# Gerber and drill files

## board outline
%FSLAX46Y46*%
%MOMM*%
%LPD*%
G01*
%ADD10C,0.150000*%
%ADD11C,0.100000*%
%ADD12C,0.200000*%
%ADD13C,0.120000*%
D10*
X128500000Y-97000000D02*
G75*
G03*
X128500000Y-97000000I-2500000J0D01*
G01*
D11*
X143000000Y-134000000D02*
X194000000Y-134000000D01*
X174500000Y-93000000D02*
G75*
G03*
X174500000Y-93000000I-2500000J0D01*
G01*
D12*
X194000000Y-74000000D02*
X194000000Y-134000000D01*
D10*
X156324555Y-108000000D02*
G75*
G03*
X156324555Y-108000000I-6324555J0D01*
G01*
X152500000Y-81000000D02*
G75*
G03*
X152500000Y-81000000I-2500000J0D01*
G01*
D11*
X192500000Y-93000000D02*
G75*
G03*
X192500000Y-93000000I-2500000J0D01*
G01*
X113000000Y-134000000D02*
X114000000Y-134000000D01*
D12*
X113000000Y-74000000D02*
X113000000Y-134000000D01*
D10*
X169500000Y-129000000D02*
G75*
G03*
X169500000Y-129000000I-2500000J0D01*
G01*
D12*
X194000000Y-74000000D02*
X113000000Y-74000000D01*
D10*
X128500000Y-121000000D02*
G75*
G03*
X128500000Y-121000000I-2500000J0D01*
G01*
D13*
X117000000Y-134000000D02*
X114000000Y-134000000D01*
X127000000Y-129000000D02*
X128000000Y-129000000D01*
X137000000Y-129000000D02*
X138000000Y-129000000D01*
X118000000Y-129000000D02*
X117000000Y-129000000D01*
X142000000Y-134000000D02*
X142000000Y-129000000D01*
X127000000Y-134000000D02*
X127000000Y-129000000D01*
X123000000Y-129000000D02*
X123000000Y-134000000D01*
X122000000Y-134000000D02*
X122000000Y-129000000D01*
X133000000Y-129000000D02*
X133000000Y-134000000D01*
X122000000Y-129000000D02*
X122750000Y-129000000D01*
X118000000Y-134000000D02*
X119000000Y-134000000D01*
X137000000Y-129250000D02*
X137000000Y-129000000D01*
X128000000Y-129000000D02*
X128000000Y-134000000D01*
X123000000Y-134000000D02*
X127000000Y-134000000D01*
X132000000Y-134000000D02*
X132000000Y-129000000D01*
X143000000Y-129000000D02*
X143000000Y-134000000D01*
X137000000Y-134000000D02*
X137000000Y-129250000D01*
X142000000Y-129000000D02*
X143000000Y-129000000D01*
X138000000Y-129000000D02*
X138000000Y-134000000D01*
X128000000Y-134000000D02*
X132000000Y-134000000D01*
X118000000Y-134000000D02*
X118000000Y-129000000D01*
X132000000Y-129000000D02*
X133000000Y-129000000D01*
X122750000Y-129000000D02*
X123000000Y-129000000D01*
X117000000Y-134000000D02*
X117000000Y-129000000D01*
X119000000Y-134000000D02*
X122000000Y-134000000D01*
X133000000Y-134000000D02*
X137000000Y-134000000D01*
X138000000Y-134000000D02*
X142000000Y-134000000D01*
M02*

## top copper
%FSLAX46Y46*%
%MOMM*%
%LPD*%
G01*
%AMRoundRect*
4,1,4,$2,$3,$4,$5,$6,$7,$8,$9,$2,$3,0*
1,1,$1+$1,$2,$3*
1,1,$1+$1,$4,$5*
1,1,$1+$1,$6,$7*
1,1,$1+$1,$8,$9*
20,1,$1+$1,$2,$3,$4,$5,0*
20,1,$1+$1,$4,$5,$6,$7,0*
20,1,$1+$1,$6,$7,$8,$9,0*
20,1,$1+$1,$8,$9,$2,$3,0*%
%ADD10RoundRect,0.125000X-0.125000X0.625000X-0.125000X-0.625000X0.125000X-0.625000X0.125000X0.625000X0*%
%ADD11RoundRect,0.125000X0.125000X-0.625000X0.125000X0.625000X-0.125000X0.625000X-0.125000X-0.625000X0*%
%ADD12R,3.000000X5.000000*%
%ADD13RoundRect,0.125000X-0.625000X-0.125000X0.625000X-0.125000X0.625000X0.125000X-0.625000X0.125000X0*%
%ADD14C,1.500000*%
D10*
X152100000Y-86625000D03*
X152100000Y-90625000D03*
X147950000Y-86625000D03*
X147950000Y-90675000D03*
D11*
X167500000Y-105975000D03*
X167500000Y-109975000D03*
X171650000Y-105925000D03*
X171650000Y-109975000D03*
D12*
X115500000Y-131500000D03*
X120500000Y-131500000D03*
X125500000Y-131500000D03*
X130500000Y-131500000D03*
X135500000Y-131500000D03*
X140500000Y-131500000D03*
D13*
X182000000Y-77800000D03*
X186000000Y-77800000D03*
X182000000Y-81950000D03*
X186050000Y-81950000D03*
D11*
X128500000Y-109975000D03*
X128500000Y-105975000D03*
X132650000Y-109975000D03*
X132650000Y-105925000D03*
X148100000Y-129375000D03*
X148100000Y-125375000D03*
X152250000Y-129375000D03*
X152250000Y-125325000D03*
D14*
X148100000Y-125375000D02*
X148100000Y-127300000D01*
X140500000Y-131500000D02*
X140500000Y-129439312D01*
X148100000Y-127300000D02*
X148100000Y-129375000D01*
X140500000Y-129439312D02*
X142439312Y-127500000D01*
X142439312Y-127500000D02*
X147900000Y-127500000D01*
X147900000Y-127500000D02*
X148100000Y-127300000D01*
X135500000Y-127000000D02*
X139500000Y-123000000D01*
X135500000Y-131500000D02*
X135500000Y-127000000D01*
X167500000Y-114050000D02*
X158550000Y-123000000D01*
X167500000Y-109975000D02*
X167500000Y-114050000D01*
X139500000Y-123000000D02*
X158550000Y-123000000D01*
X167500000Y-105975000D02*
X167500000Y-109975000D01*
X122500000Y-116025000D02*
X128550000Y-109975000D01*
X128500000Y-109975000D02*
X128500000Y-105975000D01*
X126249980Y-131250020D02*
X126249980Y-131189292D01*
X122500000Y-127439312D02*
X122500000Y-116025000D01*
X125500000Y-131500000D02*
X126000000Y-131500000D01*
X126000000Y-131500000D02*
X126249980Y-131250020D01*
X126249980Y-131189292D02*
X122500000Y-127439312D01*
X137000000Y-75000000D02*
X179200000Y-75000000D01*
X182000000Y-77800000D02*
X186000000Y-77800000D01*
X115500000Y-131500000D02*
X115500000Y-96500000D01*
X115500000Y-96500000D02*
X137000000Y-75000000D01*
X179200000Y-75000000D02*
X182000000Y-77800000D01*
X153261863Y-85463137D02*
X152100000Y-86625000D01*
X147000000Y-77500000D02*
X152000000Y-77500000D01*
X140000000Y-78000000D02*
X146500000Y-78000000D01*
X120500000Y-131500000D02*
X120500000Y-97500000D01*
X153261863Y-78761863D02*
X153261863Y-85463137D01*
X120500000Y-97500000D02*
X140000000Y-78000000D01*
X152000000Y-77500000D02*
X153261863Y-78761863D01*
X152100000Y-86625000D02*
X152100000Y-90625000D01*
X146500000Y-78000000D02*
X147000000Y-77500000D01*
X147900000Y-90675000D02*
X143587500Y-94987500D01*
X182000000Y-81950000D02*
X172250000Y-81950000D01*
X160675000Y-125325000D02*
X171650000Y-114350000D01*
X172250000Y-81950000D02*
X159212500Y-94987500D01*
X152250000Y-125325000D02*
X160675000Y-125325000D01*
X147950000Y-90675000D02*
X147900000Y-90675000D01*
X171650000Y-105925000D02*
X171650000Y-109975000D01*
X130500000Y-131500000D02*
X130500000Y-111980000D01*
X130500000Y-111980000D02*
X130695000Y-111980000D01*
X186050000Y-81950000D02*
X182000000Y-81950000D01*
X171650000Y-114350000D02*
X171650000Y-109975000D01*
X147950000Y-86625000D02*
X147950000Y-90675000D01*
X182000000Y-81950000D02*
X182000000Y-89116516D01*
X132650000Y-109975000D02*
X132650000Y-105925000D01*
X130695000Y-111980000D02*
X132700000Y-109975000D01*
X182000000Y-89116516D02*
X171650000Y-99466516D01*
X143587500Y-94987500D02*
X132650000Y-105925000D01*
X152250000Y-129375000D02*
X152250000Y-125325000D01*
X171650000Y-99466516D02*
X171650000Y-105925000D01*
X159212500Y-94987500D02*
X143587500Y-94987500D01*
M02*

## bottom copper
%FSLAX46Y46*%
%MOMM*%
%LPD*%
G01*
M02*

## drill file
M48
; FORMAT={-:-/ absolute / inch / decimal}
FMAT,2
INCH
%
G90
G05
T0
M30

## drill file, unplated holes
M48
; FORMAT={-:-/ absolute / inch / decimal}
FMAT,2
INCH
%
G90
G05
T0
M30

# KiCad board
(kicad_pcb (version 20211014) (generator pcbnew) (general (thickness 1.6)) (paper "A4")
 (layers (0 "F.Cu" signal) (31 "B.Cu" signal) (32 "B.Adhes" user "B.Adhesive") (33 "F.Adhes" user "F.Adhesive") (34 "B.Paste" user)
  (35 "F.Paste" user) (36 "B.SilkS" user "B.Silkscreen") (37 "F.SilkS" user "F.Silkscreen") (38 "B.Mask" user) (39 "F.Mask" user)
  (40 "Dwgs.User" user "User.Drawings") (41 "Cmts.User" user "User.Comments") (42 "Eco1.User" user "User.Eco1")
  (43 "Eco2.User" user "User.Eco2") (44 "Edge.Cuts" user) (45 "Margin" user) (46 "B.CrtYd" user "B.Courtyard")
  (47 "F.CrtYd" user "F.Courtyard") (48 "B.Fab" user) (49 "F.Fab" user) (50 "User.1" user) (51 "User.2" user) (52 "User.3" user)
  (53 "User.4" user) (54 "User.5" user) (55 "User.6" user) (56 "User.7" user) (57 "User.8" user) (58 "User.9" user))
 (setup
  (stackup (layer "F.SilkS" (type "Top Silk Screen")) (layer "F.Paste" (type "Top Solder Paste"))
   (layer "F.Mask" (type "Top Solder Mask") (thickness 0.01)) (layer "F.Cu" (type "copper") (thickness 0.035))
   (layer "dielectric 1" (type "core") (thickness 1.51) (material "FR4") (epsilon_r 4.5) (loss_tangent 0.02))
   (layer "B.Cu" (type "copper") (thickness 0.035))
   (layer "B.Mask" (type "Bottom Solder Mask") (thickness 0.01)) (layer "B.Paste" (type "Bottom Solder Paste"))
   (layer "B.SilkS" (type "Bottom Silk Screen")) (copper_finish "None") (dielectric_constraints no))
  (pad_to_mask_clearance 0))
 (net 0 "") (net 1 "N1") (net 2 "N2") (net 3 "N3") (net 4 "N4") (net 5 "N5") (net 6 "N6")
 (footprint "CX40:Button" (layer "F.Cu") (at 144.7 97.075 -90)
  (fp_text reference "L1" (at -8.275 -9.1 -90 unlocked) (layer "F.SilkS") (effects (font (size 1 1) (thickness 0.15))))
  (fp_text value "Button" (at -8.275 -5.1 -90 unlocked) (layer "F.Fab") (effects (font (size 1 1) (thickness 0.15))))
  (pad "1" smd roundrect (at -10.45 -7.4 270) (size 1.5 0.5) (layers "F.Cu" "F.Paste" "F.Mask") (roundrect_rratio 0.25) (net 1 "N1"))
  (pad "1" smd roundrect (at -6.45 -7.4 270) (size 1.5 0.5) (layers "F.Cu" "F.Paste" "F.Mask") (roundrect_rratio 0.25) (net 1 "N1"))
  (pad "2" smd roundrect (at -10.45 -3.25 270) (size 1.5 0.5) (layers "F.Cu" "F.Paste" "F.Mask") (roundrect_rratio 0.25) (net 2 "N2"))
  (pad "2" smd roundrect (at -6.4 -3.25 270) (size 1.5 0.5) (layers "F.Cu" "F.Paste" "F.Mask") (roundrect_rratio 0.25) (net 2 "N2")))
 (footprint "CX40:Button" (layer "F.Cu") (at 174.9 99.525 90)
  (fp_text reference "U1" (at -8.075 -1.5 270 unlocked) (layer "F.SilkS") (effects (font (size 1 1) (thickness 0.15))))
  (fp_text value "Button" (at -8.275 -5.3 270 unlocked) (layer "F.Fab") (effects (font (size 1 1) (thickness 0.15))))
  (pad "1" smd roundrect (at -6.45 -7.4 90) (size 1.5 0.5) (layers "F.Cu" "F.Paste" "F.Mask") (roundrect_rratio 0.25) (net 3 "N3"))
  (pad "1" smd roundrect (at -10.45 -7.4 90) (size 1.5 0.5) (layers "F.Cu" "F.Paste" "F.Mask") (roundrect_rratio 0.25) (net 3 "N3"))
  (pad "2" smd roundrect (at -6.4 -3.25 90) (size 1.5 0.5) (layers "F.Cu" "F.Paste" "F.Mask") (roundrect_rratio 0.25) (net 2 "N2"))
  (pad "2" smd roundrect (at -10.45 -3.25 90) (size 1.5 0.5) (layers "F.Cu" "F.Paste" "F.Mask") (roundrect_rratio 0.25) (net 2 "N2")))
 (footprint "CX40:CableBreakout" (layer "F.Cu") (at 120 136)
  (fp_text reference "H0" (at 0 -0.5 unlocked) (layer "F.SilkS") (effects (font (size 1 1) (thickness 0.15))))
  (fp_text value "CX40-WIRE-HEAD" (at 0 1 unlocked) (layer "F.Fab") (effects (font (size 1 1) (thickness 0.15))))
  (fp_line (start -3 -2) (end -6 -2) (layer "Edge.Cuts") (width 0.12))
  (fp_line (start 7 -7) (end 8 -7) (layer "Edge.Cuts") (width 0.12))
  (fp_line (start 17 -7) (end 18 -7) (layer "Edge.Cuts") (width 0.12))
  (fp_line (start -2 -7) (end -3 -7) (layer "Edge.Cuts") (width 0.12))
  (fp_line (start 22 -2) (end 22 -7) (layer "Edge.Cuts") (width 0.12))
  (fp_line (start 7 -2) (end 7 -7) (layer "Edge.Cuts") (width 0.12))
  (fp_line (start 3 -7) (end 3 -2) (layer "Edge.Cuts") (width 0.12))
  (fp_line (start 2 -2) (end 2 -7) (layer "Edge.Cuts") (width 0.12))
  (fp_line (start 13 -7) (end 13 -2) (layer "Edge.Cuts") (width 0.12))
  (fp_line (start 2 -7) (end 2.75 -7) (layer "Edge.Cuts") (width 0.12))
  (fp_line (start -2 -2) (end -1 -2) (layer "Edge.Cuts") (width 0.12))
  (fp_line (start 17 -6.75) (end 17 -7) (layer "Edge.Cuts") (width 0.12))
  (fp_line (start 8 -7) (end 8 -2) (layer "Edge.Cuts") (width 0.12))
  (fp_line (start 3 -2) (end 7 -2) (layer "Edge.Cuts") (width 0.12))
  (fp_line (start 12 -2) (end 12 -7) (layer "Edge.Cuts") (width 0.12))
  (fp_line (start 23 -7) (end 23 -2) (layer "Edge.Cuts") (width 0.12))
  (fp_line (start 17 -2) (end 17 -6.75) (layer "Edge.Cuts") (width 0.12))
  (fp_line (start 22 -7) (end 23 -7) (layer "Edge.Cuts") (width 0.12))
  (fp_line (start 18 -7) (end 18 -2) (layer "Edge.Cuts") (width 0.12))
  (fp_line (start 8 -2) (end 12 -2) (layer "Edge.Cuts") (width 0.12))
  (fp_line (start -2 -2) (end -2 -7) (layer "Edge.Cuts") (width 0.12))
  (fp_line (start 12 -7) (end 13 -7) (layer "Edge.Cuts") (width 0.12))
  (fp_line (start 2.75 -7) (end 3 -7) (layer "Edge.Cuts") (width 0.12))
  (fp_line (start -3 -2) (end -3 -7) (layer "Edge.Cuts") (width 0.12))
  (fp_line (start -1 -2) (end 2 -2) (layer "Edge.Cuts") (width 0.12))
  (fp_line (start 13 -2) (end 17 -2) (layer "Edge.Cuts") (width 0.12))
  (fp_line (start 18 -2) (end 22 -2) (layer "Edge.Cuts") (width 0.12))
  (pad "1" connect rect (at -4.5 -4.5) (size 3 5) (layers "F.Cu" "F.Mask") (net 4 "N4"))
  (pad "2" connect rect (at 0.5 -4.5) (size 3 5) (layers "F.Cu" "F.Mask") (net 1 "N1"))
  (pad "3" connect rect (at 5.5 -4.5) (size 3 5) (layers "F.Cu" "F.Mask") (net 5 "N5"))
  (pad "4" connect rect (at 10.5 -4.5) (size 3 5) (layers "F.Cu" "F.Mask") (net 2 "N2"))
  (pad "5" connect rect (at 15.5 -4.5) (size 3 5) (layers "F.Cu" "F.Mask") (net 3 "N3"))
  (pad "6" connect rect (at 20.5 -4.5) (size 3 5) (layers "F.Cu" "F.Mask") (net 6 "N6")))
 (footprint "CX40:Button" (layer "F.Cu") (at 192.45 85.2)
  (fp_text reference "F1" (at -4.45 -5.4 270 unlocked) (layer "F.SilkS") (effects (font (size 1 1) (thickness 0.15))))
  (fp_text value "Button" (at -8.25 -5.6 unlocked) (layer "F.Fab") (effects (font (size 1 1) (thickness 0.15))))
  (pad "1" smd roundrect (at -10.45 -7.4) (size 1.5 0.5) (layers "F.Cu" "F.Paste" "F.Mask") (roundrect_rratio 0.25) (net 4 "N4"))
  (pad "1" smd roundrect (at -6.45 -7.4) (size 1.5 0.5) (layers "F.Cu" "F.Paste" "F.Mask") (roundrect_rratio 0.25) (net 4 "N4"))
  (pad "2" smd roundrect (at -10.45 -3.25) (size 1.5 0.5) (layers "F.Cu" "F.Paste" "F.Mask") (roundrect_rratio 0.25) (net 2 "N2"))
  (pad "2" smd roundrect (at -6.4 -3.25) (size 1.5 0.5) (layers "F.Cu" "F.Paste" "F.Mask") (roundrect_rratio 0.25) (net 2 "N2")))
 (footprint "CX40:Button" (layer "F.Cu") (at 135.9 99.525 90)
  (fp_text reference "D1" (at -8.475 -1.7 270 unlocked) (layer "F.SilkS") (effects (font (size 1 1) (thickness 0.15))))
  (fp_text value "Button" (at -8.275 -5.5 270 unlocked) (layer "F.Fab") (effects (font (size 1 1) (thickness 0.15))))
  (pad "1" smd roundrect (at -10.45 -7.4 90) (size 1.5 0.5) (layers "F.Cu" "F.Paste" "F.Mask") (roundrect_rratio 0.25) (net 5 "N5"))
  (pad "1" smd roundrect (at -6.45 -7.4 90) (size 1.5 0.5) (layers "F.Cu" "F.Paste" "F.Mask") (roundrect_rratio 0.25) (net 5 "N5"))
  (pad "2" smd roundrect (at -10.45 -3.25 90) (size 1.5 0.5) (layers "F.Cu" "F.Paste" "F.Mask") (roundrect_rratio 0.25) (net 2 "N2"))
  (pad "2" smd roundrect (at -6.4 -3.25 90) (size 1.5 0.5) (layers "F.Cu" "F.Paste" "F.Mask") (roundrect_rratio 0.25) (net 2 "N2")))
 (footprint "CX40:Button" (layer "F.Cu") (at 155.5 118.925 90)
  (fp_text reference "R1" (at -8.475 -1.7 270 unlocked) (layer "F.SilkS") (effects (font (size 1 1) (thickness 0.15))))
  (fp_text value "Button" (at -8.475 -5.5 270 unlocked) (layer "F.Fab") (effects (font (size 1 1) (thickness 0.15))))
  (pad "1" smd roundrect (at -10.45 -7.4 90) (size 1.5 0.5) (layers "F.Cu" "F.Paste" "F.Mask") (roundrect_rratio 0.25) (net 6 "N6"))
  (pad "1" smd roundrect (at -6.45 -7.4 90) (size 1.5 0.5) (layers "F.Cu" "F.Paste" "F.Mask") (roundrect_rratio 0.25) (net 6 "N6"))
  (pad "2" smd roundrect (at -10.45 -3.25 90) (size 1.5 0.5) (layers "F.Cu" "F.Paste" "F.Mask") (roundrect_rratio 0.25) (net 2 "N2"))
  (pad "2" smd roundrect (at -6.4 -3.25 90) (size 1.5 0.5) (layers "F.Cu" "F.Paste" "F.Mask") (roundrect_rratio 0.25) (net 2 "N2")))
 (gr_circle (center 126 97) (end 128.5 97) (layer "Edge.Cuts") (width 0.15) (fill none))
 (gr_line (start 143 134) (end 194 134) (layer "Edge.Cuts") (width 0.1))
 (gr_circle (center 172 93) (end 174.5 93) (layer "Edge.Cuts") (width 0.1) (fill none))
 (gr_line (start 194 74) (end 194 134) (layer "Edge.Cuts") (width 0.2))
 (gr_circle (center 150 108) (end 156.324555 108) (layer "Edge.Cuts") (width 0.15) (fill none))
 (gr_circle (center 150 81) (end 152.5 81) (layer "Edge.Cuts") (width 0.15) (fill none))
 (gr_circle (center 190 93) (end 192.5 93) (layer "Edge.Cuts") (width 0.1) (fill none))
 (gr_line (start 113 134) (end 114 134) (layer "Edge.Cuts") (width 0.1))
 (gr_line (start 113 74) (end 113 134) (layer "Edge.Cuts") (width 0.2))
 (gr_circle (center 167 129) (end 169.5 129) (layer "Edge.Cuts") (width 0.15) (fill none))
 (gr_line (start 194 74) (end 113 74) (layer "Edge.Cuts") (width 0.2))
 (gr_circle (center 126 121) (end 128.5 121) (layer "Edge.Cuts") (width 0.15) (fill none))
 (segment (start 135.5 127) (end 139.5 123) (width 1.5) (layer "F.Cu") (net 3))
 (segment (start 135.5 131.5) (end 135.5 127) (width 1.5) (layer "F.Cu") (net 3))
 (segment (start 167.5 114.05) (end 158.55 123) (width 1.5) (layer "F.Cu") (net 3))
 (segment (start 167.5 109.975) (end 167.5 114.05) (width 1.5) (layer "F.Cu") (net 3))
 (segment (start 139.5 123) (end 158.55 123) (width 1.5) (layer "F.Cu") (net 3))
 (segment (start 167.5 105.975) (end 167.5 109.975) (width 1.5) (layer "F.Cu") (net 3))
 (segment (start 140.5 131.5) (end 140.5 129.439312) (width 1.5) (layer "F.Cu") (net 6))
 (segment (start 142.439312 127.5) (end 147.9 127.5) (width 1.5) (layer "F.Cu") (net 6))
 (segment (start 140.5 129.439312) (end 142.439312 127.5) (width 1.5) (layer "F.Cu") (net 6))
 (segment (start 148.1 125.375) (end 148.1 127.3) (width 1.5) (layer "F.Cu") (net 6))
 (segment (start 147.9 127.5) (end 148.1 127.3) (width 1.5) (layer "F.Cu") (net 6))
 (segment (start 148.1 127.3) (end 148.1 129.375) (width 1.5) (layer "F.Cu") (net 6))
 (segment (start 122.5 116.025) (end 128.55 109.975) (width 1.5) (layer "F.Cu") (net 5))
 (segment (start 128.5 109.975) (end 128.5 105.975) (width 1.5) (layer "F.Cu") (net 5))
 (segment (start 126.24998 131.25002) (end 126.24998 131.189292) (width 1.5) (layer "F.Cu") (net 5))
 (segment (start 122.5 127.439312) (end 122.5 116.025) (width 1.5) (layer "F.Cu") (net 5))
 (segment (start 125.5 131.5) (end 126 131.5) (width 1.5) (layer "F.Cu") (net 5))
 (segment (start 126 131.5) (end 126.24998 131.25002) (width 1.5) (layer "F.Cu") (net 5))
 (segment (start 126.24998 131.189292) (end 122.5 127.439312) (width 1.5) (layer "F.Cu") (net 5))
 (segment (start 137 75) (end 179.2 75) (width 1.5) (layer "F.Cu") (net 4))
 (segment (start 182 77.8) (end 186 77.8) (width 1.5) (layer "F.Cu") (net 4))
 (segment (start 115.5 131.5) (end 115.5 96.5) (width 1.5) (layer "F.Cu") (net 4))
 (segment (start 115.5 96.5) (end 137 75) (width 1.5) (layer "F.Cu") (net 4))
 (segment (start 179.2 75) (end 182 77.8) (width 1.5) (layer "F.Cu") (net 4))
 (segment (start 153.261863 85.463137) (end 152.1 86.625) (width 1.5) (layer "F.Cu") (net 1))
 (segment (start 147 77.5) (end 152 77.5) (width 1.5) (layer "F.Cu") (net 1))
 (segment (start 140 78) (end 146.5 78) (width 1.5) (layer "F.Cu") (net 1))
 (segment (start 120.5 131.5) (end 120.5 97.5) (width 1.5) (layer "F.Cu") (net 1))
 (segment (start 153.261863 78.761863) (end 153.261863 85.463137) (width 1.5) (layer "F.Cu") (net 1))
 (segment (start 120.5 97.5) (end 140 78) (width 1.5) (layer "F.Cu") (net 1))
 (segment (start 152 77.5) (end 153.261863 78.761863) (width 1.5) (layer "F.Cu") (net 1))
 (segment (start 152.1 86.625) (end 152.1 90.625) (width 1.5) (layer "F.Cu") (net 1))
 (segment (start 146.5 78) (end 147 77.5) (width 1.5) (layer "F.Cu") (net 1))
 (segment (start 147.9 90.675) (end 143.5875 94.9875) (width 1.5) (layer "F.Cu") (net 2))
 (segment (start 182 81.95) (end 172.25 81.95) (width 1.5) (layer "F.Cu") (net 2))
 (segment (start 160.675 125.325) (end 171.65 114.35) (width 1.5) (layer "F.Cu") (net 2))
 (segment (start 172.25 81.95) (end 159.2125 94.9875) (width 1.5) (layer "F.Cu") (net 2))
 (segment (start 152.25 125.325) (end 160.675 125.325) (width 1.5) (layer "F.Cu") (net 2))
 (segment (start 147.95 90.675) (end 147.9 90.675) (width 1.5) (layer "F.Cu") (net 2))
 (segment (start 171.65 105.925) (end 171.65 109.975) (width 1.5) (layer "F.Cu") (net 2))
 (segment (start 130.5 131.5) (end 130.5 111.98) (width 1.5) (layer "F.Cu") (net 2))
 (segment (start 130.5 111.98) (end 130.695 111.98) (width 1.5) (layer "F.Cu") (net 2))
 (segment (start 186.05 81.95) (end 182 81.95) (width 1.5) (layer "F.Cu") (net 2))
 (segment (start 171.65 114.35) (end 171.65 109.975) (width 1.5) (layer "F.Cu") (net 2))
 (segment (start 147.95 86.625) (end 147.95 90.675) (width 1.5) (layer "F.Cu") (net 2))
 (segment (start 182 81.95) (end 182 89.116516) (width 1.5) (layer "F.Cu") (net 2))
 (segment (start 132.65 109.975) (end 132.65 105.925) (width 1.5) (layer "F.Cu") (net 2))
 (segment (start 130.695 111.98) (end 132.7 109.975) (width 1.5) (layer "F.Cu") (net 2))
 (segment (start 182 89.116516) (end 171.65 99.466516) (width 1.5) (layer "F.Cu") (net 2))
 (segment (start 143.5875 94.9875) (end 132.65 105.925) (width 1.5) (layer "F.Cu") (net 2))
 (segment (start 152.25 129.375) (end 152.25 125.325) (width 1.5) (layer "F.Cu") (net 2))
 (segment (start 171.65 99.466516) (end 171.65 105.925) (width 1.5) (layer "F.Cu") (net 2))
 (segment (start 159.2125 94.9875) (end 143.5875 94.9875) (width 1.5) (layer "F.Cu") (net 2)))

